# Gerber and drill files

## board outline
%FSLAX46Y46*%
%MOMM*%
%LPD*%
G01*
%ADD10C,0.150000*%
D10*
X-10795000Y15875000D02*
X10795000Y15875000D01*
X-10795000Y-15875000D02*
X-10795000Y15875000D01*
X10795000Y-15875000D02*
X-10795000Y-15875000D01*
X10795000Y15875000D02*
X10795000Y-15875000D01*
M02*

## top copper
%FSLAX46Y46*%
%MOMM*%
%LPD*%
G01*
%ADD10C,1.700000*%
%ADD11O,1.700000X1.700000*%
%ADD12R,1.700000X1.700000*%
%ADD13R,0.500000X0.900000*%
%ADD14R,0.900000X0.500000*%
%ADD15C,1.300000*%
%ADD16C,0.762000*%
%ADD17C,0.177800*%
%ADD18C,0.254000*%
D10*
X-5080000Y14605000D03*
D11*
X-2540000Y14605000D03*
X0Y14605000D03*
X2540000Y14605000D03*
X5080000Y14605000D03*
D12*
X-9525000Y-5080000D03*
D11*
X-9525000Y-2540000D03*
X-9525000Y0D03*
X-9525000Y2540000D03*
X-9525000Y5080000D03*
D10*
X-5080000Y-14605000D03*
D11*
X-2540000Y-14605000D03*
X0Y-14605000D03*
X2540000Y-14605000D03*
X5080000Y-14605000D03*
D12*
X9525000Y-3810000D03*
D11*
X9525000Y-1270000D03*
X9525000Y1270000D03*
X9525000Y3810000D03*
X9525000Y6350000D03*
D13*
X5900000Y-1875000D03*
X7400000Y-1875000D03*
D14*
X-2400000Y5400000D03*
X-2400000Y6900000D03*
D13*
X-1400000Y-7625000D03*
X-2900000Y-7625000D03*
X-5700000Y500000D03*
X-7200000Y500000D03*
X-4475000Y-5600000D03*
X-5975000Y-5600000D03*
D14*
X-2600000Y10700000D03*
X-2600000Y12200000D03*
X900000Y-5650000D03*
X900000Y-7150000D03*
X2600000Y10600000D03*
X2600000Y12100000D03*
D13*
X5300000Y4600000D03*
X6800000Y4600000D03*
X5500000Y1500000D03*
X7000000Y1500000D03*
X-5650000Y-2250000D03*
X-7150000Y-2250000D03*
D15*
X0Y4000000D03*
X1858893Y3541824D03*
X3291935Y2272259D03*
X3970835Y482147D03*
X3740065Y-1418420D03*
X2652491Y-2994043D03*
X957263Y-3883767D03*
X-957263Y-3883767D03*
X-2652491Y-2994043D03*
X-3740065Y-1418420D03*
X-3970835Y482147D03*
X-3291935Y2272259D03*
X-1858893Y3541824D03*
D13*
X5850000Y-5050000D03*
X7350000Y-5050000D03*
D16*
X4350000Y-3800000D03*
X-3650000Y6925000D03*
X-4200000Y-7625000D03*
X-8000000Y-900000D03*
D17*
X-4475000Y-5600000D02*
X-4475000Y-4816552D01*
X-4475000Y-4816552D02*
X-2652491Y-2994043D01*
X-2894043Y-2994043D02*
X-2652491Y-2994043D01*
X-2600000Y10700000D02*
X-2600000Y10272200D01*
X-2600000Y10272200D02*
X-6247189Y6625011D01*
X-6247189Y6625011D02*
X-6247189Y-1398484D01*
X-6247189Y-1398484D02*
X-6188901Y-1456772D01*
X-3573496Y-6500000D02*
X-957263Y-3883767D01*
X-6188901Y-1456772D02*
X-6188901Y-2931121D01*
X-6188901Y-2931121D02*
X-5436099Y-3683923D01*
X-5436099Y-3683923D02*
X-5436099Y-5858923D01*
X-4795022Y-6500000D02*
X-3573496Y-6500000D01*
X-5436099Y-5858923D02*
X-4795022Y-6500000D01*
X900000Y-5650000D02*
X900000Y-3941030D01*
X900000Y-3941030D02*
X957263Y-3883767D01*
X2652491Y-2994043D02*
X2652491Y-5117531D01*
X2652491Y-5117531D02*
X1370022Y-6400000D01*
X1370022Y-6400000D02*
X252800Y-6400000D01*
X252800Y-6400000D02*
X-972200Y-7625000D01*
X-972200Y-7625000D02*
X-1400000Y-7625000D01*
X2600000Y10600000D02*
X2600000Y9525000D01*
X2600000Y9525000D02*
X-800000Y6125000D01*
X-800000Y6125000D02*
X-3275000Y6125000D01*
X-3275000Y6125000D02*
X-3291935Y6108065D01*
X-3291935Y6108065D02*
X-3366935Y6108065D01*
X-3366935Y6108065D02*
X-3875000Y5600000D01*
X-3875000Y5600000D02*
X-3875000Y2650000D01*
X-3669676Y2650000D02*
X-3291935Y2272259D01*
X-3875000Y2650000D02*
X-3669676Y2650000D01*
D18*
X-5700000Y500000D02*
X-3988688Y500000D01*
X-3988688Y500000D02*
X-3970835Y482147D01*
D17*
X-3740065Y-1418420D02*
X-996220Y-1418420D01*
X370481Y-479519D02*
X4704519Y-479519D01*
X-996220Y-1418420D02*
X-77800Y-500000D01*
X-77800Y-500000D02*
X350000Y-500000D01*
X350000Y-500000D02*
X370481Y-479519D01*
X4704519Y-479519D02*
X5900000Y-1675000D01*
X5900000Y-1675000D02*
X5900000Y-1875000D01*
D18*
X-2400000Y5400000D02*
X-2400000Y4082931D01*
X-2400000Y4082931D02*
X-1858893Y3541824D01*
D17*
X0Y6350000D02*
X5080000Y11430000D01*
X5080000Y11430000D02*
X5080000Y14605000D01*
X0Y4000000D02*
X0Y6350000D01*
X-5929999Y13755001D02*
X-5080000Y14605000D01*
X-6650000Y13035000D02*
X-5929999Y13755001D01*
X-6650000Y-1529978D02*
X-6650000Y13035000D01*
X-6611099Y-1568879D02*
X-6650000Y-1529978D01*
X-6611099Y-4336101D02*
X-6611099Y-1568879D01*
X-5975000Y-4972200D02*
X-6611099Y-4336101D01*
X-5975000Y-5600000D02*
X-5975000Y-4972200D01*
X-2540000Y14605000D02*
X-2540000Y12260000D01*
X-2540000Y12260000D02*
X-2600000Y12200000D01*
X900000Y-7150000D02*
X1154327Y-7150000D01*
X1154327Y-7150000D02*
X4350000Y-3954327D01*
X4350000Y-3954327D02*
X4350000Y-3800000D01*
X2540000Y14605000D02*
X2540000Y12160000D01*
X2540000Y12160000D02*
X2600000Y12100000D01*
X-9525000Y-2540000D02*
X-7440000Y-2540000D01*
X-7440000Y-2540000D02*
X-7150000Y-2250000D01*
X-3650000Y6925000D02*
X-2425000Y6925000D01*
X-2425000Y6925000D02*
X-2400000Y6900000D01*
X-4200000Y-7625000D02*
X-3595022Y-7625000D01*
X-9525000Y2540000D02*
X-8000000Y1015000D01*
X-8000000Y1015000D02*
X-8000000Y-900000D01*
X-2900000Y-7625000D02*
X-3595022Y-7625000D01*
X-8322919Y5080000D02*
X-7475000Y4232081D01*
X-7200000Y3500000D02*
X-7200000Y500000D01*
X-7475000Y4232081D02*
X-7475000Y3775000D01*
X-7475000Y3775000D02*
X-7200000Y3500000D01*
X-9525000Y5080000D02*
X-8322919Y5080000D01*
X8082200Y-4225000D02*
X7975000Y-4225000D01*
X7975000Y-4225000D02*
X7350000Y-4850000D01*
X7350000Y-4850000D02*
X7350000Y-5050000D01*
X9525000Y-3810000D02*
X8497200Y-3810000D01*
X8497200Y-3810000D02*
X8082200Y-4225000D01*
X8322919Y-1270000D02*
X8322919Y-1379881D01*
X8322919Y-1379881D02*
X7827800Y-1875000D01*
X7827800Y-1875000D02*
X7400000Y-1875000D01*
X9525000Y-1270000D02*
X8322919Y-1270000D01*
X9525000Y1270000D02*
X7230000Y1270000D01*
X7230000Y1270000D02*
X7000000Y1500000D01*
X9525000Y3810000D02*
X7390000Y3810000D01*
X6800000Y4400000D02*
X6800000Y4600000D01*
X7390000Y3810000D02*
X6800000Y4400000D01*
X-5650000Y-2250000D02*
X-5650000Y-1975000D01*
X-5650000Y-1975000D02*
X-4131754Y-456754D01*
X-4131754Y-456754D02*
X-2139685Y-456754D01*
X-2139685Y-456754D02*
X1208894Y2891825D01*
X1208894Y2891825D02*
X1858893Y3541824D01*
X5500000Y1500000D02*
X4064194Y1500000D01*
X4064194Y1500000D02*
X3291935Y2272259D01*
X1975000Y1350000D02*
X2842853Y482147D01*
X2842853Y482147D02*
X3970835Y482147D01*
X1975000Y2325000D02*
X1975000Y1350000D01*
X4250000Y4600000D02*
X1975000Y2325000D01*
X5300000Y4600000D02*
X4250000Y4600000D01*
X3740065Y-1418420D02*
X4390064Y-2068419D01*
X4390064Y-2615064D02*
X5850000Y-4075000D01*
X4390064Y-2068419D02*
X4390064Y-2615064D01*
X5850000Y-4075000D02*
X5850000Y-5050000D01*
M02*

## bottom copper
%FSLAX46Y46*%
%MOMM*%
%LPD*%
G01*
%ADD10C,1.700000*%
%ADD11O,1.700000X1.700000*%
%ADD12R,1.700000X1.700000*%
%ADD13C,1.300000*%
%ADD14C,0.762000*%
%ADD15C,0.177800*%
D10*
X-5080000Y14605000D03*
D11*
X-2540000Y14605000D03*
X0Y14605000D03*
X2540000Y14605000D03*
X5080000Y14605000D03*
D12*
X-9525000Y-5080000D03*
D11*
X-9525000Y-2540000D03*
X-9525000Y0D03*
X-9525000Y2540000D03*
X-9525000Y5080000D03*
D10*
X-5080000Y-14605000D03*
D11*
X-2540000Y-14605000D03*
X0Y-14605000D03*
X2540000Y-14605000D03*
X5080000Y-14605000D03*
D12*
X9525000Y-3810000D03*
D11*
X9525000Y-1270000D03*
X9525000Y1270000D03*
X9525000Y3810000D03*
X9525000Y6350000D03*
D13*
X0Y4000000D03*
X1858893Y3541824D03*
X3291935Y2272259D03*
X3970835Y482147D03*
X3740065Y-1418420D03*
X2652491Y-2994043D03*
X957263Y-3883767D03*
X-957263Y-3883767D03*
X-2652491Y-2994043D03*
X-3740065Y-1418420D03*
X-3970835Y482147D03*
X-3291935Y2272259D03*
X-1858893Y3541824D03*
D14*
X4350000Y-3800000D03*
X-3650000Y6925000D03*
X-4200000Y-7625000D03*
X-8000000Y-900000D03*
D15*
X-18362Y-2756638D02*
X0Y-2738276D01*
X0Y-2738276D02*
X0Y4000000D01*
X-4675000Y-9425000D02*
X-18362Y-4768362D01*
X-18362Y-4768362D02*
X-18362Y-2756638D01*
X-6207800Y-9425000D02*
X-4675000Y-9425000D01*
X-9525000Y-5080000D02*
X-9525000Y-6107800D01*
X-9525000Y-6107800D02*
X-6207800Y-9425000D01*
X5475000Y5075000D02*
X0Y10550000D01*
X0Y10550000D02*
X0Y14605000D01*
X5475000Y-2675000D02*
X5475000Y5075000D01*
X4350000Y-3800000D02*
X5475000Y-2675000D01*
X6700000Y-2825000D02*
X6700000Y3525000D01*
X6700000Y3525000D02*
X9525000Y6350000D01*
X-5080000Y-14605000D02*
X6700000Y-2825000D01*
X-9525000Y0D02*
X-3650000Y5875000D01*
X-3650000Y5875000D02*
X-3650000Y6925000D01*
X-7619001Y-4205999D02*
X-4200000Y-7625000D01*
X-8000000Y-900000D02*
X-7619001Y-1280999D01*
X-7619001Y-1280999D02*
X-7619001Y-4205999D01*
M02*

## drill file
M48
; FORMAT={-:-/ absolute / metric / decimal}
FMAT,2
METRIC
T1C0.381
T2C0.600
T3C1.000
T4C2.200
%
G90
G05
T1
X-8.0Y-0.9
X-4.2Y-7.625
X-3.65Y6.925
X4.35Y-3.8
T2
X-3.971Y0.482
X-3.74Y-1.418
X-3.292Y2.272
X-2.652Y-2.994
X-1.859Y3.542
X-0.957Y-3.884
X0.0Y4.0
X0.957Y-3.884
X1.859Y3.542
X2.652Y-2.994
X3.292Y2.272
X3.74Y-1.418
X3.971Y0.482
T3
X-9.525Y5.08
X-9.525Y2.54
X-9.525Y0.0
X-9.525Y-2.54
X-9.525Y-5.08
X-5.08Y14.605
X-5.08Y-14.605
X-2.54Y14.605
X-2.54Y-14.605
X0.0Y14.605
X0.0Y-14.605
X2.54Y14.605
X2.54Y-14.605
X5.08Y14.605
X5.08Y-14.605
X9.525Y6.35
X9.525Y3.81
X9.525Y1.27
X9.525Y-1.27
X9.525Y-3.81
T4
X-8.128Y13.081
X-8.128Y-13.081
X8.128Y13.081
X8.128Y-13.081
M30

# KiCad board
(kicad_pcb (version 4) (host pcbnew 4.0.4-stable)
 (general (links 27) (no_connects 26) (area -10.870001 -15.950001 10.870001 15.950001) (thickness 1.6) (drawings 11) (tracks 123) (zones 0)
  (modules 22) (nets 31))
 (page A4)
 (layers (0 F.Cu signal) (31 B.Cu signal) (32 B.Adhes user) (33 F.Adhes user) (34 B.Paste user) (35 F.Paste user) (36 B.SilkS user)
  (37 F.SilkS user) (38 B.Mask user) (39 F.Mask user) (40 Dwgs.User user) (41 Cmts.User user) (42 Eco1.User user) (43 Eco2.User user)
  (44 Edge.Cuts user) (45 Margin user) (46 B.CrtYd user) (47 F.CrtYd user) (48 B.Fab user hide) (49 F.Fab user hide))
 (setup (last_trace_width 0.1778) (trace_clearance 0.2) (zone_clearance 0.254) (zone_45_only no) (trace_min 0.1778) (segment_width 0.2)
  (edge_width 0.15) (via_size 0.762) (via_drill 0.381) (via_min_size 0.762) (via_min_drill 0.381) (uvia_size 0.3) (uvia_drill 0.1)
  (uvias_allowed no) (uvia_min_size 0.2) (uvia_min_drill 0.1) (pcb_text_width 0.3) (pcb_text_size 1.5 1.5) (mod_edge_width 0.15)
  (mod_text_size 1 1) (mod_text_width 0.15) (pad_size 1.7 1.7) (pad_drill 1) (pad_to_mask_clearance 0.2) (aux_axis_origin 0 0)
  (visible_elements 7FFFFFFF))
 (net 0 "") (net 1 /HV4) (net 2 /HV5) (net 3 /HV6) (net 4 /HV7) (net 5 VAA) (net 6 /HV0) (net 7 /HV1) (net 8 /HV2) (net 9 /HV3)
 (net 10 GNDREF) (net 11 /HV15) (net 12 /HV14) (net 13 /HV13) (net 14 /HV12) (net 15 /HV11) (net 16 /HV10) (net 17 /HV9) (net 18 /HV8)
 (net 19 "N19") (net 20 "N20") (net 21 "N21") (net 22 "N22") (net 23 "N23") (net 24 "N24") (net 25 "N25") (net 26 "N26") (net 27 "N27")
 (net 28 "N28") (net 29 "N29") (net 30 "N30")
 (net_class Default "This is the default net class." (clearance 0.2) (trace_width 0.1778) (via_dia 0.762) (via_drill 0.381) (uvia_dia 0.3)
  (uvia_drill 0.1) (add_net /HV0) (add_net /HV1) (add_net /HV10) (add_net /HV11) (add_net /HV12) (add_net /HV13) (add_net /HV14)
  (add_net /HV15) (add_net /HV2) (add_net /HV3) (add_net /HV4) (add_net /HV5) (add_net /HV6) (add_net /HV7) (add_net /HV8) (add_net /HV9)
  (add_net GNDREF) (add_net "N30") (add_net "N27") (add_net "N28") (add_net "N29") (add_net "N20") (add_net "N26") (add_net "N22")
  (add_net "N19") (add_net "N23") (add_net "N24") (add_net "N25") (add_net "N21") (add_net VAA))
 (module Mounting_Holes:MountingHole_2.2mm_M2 (layer F.Cu) (at 8.128 13.081)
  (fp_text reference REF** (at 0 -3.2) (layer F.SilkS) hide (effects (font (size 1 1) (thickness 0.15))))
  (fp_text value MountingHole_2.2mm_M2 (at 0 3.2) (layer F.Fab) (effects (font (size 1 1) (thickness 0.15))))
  (pad 1 np_thru_hole circle (at 0 0) (size 2.2 2.2) (drill 2.2) (layers *.Cu *.Mask)))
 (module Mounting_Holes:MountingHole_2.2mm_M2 (layer F.Cu) (at 8.128 -13.081)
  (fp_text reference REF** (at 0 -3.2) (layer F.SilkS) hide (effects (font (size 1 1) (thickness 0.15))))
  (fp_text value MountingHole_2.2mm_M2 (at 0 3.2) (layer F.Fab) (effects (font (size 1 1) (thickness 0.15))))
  (pad 1 np_thru_hole circle (at 0 0) (size 2.2 2.2) (drill 2.2) (layers *.Cu *.Mask)))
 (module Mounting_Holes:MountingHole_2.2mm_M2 (layer F.Cu) (at -8.128 -13.081)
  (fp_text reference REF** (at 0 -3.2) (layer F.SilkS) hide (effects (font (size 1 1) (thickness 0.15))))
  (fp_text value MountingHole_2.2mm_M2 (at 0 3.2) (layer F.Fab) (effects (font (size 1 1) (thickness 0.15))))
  (pad 1 np_thru_hole circle (at 0 0) (size 2.2 2.2) (drill 2.2) (layers *.Cu *.Mask)))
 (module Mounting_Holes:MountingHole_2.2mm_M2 (layer F.Cu) (at -8.128 13.081)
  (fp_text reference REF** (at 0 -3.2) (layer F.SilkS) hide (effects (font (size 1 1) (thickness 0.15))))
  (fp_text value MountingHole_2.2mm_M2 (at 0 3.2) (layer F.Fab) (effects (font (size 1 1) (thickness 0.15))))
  (pad 1 np_thru_hole circle (at 0 0) (size 2.2 2.2) (drill 2.2) (layers *.Cu *.Mask)))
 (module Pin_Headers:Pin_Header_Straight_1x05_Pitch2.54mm (layer F.Cu) (at -5.08 -14.605 90)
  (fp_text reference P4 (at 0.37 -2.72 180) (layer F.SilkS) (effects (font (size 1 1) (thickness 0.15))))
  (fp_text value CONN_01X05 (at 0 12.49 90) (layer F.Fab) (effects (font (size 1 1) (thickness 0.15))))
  (pad 1 thru_hole circle (at 0 0 90) (size 1.7 1.7) (drill 1) (layers *.Cu *.Mask) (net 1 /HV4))
  (pad 2 thru_hole oval (at 0 2.54 90) (size 1.7 1.7) (drill 1) (layers *.Cu *.Mask) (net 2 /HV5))
  (pad 3 thru_hole oval (at 0 5.08 90) (size 1.7 1.7) (drill 1) (layers *.Cu *.Mask) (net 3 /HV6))
  (pad 4 thru_hole oval (at 0 7.62 90) (size 1.7 1.7) (drill 1) (layers *.Cu *.Mask) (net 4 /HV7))
  (pad 5 thru_hole oval (at 0 10.16 90) (size 1.7 1.7) (drill 1) (layers *.Cu *.Mask) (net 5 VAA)))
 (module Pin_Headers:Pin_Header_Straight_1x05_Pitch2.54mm (layer F.Cu) (at -9.525 5.08 180)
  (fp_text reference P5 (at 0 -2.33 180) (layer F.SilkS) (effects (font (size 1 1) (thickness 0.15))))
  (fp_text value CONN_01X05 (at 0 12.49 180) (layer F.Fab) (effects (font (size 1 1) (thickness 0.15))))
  (pad 1 thru_hole rect (at 0 0 180) (size 1.7 1.7) (drill 1) (layers *.Cu *.Mask) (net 5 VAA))
  (pad 2 thru_hole oval (at 0 2.54 180) (size 1.7 1.7) (drill 1) (layers *.Cu *.Mask) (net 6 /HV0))
  (pad 3 thru_hole oval (at 0 5.08 180) (size 1.7 1.7) (drill 1) (layers *.Cu *.Mask) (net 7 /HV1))
  (pad 4 thru_hole oval (at 0 7.62 180) (size 1.7 1.7) (drill 1) (layers *.Cu *.Mask) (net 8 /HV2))
  (pad 5 thru_hole oval (at 0 10.16 180) (size 1.7 1.7) (drill 1) (layers *.Cu *.Mask) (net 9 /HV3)))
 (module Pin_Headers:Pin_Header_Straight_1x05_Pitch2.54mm (layer F.Cu) (at -5.08 14.605 90)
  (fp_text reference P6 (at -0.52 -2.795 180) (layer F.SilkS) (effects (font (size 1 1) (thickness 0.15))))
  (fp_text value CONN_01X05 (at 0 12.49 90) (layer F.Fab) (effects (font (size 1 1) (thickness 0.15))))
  (pad 1 thru_hole circle (at 0 0 90) (size 1.7 1.7) (drill 1) (layers *.Cu *.Mask) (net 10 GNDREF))
  (pad 2 thru_hole oval (at 0 2.54 90) (size 1.7 1.7) (drill 1) (layers *.Cu *.Mask) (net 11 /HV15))
  (pad 3 thru_hole oval (at 0 5.08 90) (size 1.7 1.7) (drill 1) (layers *.Cu *.Mask) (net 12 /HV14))
  (pad 4 thru_hole oval (at 0 7.62 90) (size 1.7 1.7) (drill 1) (layers *.Cu *.Mask) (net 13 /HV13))
  (pad 5 thru_hole oval (at 0 10.16 90) (size 1.7 1.7) (drill 1) (layers *.Cu *.Mask) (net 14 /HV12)))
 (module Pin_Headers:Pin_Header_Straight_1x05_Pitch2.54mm (layer F.Cu) (at 9.525 3.81 180)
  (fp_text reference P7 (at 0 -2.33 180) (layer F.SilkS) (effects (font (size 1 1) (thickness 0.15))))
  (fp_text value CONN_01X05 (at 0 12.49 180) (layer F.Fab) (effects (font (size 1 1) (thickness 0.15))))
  (pad 1 thru_hole rect (at 0 0 180) (size 1.7 1.7) (drill 1) (layers *.Cu *.Mask) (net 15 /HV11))
  (pad 2 thru_hole oval (at 0 2.54 180) (size 1.7 1.7) (drill 1) (layers *.Cu *.Mask) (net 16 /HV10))
  (pad 3 thru_hole oval (at 0 5.08 180) (size 1.7 1.7) (drill 1) (layers *.Cu *.Mask) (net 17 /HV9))
  (pad 4 thru_hole oval (at 0 7.62 180) (size 1.7 1.7) (drill 1) (layers *.Cu *.Mask) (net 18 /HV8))
  (pad 5 thru_hole oval (at 0 10.16 180) (size 1.7 1.7) (drill 1) (layers *.Cu *.Mask) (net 10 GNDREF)))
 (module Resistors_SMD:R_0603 (layer F.Cu) (at 6.65 1.875)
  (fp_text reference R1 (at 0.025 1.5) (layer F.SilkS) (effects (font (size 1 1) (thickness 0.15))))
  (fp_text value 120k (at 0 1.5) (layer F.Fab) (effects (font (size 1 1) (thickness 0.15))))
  (pad 1 smd rect (at -0.75 0) (size 0.5 0.9) (layers F.Cu F.Paste F.Mask) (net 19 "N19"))
  (pad 2 smd rect (at 0.75 0) (size 0.5 0.9) (layers F.Cu F.Paste F.Mask) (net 16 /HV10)))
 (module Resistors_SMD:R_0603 (layer F.Cu) (at -2.4 -6.15 90)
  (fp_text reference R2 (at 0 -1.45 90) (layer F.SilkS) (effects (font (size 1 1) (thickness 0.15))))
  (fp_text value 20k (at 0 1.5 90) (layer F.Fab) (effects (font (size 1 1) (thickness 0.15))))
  (pad 1 smd rect (at -0.75 0 90) (size 0.5 0.9) (layers F.Cu F.Paste F.Mask) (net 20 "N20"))
  (pad 2 smd rect (at 0.75 0 90) (size 0.5 0.9) (layers F.Cu F.Paste F.Mask) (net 7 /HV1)))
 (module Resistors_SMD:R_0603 (layer F.Cu) (at -2.15 7.625 180)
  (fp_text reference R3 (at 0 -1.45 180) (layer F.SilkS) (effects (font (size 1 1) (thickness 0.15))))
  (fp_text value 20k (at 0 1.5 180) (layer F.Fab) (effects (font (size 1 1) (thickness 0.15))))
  (pad 1 smd rect (at -0.75 0 180) (size 0.5 0.9) (layers F.Cu F.Paste F.Mask) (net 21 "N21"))
  (pad 2 smd rect (at 0.75 0 180) (size 0.5 0.9) (layers F.Cu F.Paste F.Mask) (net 8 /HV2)))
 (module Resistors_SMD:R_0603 (layer F.Cu) (at -6.45 -0.5 180)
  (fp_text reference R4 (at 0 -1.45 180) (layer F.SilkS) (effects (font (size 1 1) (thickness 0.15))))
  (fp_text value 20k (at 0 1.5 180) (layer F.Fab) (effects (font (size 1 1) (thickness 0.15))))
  (pad 1 smd rect (at -0.75 0 180) (size 0.5 0.9) (layers F.Cu F.Paste F.Mask) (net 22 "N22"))
  (pad 2 smd rect (at 0.75 0 180) (size 0.5 0.9) (layers F.Cu F.Paste F.Mask) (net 9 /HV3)))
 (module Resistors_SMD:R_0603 (layer F.Cu) (at -5.225 5.6 180)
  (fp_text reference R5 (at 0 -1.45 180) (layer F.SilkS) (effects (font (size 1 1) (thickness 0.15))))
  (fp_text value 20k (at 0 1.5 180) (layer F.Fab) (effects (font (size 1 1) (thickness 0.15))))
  (pad 1 smd rect (at -0.75 0 180) (size 0.5 0.9) (layers F.Cu F.Paste F.Mask) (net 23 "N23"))
  (pad 2 smd rect (at 0.75 0 180) (size 0.5 0.9) (layers F.Cu F.Paste F.Mask) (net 1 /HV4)))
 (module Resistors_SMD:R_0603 (layer F.Cu) (at -2.6 -11.45 90)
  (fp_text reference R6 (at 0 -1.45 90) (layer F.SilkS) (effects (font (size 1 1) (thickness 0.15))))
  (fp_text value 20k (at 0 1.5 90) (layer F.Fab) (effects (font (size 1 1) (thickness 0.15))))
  (pad 1 smd rect (at -0.75 0 90) (size 0.5 0.9) (layers F.Cu F.Paste F.Mask) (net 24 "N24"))
  (pad 2 smd rect (at 0.75 0 90) (size 0.5 0.9) (layers F.Cu F.Paste F.Mask) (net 2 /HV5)))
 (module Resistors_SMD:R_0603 (layer F.Cu) (at 0.9 6.4 270)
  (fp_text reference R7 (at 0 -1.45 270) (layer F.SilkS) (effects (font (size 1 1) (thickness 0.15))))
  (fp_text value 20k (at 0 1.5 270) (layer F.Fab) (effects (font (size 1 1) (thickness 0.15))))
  (pad 1 smd rect (at -0.75 0 270) (size 0.5 0.9) (layers F.Cu F.Paste F.Mask) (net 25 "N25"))
  (pad 2 smd rect (at 0.75 0 270) (size 0.5 0.9) (layers F.Cu F.Paste F.Mask) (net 3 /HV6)))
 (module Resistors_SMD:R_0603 (layer F.Cu) (at 2.6 -11.35 90)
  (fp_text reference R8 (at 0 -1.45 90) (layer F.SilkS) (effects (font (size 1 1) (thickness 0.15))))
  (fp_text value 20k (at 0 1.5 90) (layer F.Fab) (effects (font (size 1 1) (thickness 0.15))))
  (pad 1 smd rect (at -0.75 0 90) (size 0.5 0.9) (layers F.Cu F.Paste F.Mask) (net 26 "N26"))
  (pad 2 smd rect (at 0.75 0 90) (size 0.5 0.9) (layers F.Cu F.Paste F.Mask) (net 4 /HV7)))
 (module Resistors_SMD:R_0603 (layer F.Cu) (at 6.05 -4.6)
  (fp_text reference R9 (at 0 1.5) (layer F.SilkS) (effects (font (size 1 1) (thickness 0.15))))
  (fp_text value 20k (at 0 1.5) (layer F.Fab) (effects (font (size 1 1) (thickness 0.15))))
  (pad 1 smd rect (at -0.75 0) (size 0.5 0.9) (layers F.Cu F.Paste F.Mask) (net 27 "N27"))
  (pad 2 smd rect (at 0.75 0) (size 0.5 0.9) (layers F.Cu F.Paste F.Mask) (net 18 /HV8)))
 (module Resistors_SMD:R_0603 (layer F.Cu) (at 6.25 -1.5)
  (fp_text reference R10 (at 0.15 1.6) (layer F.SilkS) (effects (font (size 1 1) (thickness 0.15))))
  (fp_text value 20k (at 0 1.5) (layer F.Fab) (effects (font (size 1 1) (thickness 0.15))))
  (pad 1 smd rect (at -0.75 0) (size 0.5 0.9) (layers F.Cu F.Paste F.Mask) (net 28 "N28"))
  (pad 2 smd rect (at 0.75 0) (size 0.5 0.9) (layers F.Cu F.Paste F.Mask) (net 17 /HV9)))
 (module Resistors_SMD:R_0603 (layer F.Cu) (at -6.4 2.25 180)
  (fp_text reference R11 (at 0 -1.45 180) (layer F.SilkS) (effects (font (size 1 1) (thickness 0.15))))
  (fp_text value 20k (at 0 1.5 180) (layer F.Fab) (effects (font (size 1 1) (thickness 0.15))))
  (pad 1 smd rect (at -0.75 0 180) (size 0.5 0.9) (layers F.Cu F.Paste F.Mask) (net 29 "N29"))
  (pad 2 smd rect (at 0.75 0 180) (size 0.5 0.9) (layers F.Cu F.Paste F.Mask) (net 6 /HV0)))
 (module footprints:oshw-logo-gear (layer B.Cu) (at 6.9342 -9.652 180)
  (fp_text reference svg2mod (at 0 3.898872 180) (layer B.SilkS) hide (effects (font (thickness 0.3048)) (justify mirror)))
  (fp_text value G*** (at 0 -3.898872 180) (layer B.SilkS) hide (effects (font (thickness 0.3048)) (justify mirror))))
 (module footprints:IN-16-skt (layer B.Cu) (at 0 0 180)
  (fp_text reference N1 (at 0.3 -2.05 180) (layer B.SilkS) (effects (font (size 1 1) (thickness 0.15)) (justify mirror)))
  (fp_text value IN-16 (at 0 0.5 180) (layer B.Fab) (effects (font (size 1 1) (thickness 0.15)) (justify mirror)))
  (pad 1 thru_hole circle (at 0 4 180) (size 1.3 1.3) (drill 0.6) (layers *.Cu *.Mask) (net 5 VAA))
  (pad 13 thru_hole circle (at -1.858893 3.541824 152.3077) (size 1.3 1.3) (drill 0.6) (layers *.Cu *.Mask) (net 29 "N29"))
  (pad 12 thru_hole circle (at -3.291935 2.272259 124.6154) (size 1.3 1.3) (drill 0.6) (layers *.Cu *.Mask) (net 28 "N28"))
  (pad 11 thru_hole circle (at -3.970835 0.482147 96.9231) (size 1.3 1.3) (drill 0.6) (layers *.Cu *.Mask) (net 27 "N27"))
  (pad 10 thru_hole circle (at -3.740065 -1.41842 69.231) (size 1.3 1.3) (drill 0.6) (layers *.Cu *.Mask) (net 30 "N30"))
  (pad 9 thru_hole circle (at -2.652491 -2.994043 41.538) (size 1.3 1.3) (drill 0.6) (layers *.Cu *.Mask) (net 21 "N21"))
  (pad 8 thru_hole circle (at -0.957263 -3.883767 13.846) (size 1.3 1.3) (drill 0.6) (layers *.Cu *.Mask) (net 25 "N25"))
  (pad 7 thru_hole circle (at 0.957263 -3.883767 346.154) (size 1.3 1.3) (drill 0.6) (layers *.Cu *.Mask) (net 24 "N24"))
  (pad 6 thru_hole circle (at 2.652491 -2.994043 318.462) (size 1.3 1.3) (drill 0.6) (layers *.Cu *.Mask) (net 23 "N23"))
  (pad 5 thru_hole circle (at 3.740065 -1.41842 290.769) (size 1.3 1.3) (drill 0.6) (layers *.Cu *.Mask) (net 19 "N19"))
  (pad 4 thru_hole circle (at 3.970835 0.482147 263.0769) (size 1.3 1.3) (drill 0.6) (layers *.Cu *.Mask) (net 22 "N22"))
  (pad 3 thru_hole circle (at 3.291935 2.272259 235.3846) (size 1.3 1.3) (drill 0.6) (layers *.Cu *.Mask) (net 26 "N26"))
  (pad 2 thru_hole circle (at 1.858893 3.541824 207.6923) (size 1.3 1.3) (drill 0.6) (layers *.Cu *.Mask) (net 20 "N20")))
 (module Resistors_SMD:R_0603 (layer F.Cu) (at 6.6 5.05)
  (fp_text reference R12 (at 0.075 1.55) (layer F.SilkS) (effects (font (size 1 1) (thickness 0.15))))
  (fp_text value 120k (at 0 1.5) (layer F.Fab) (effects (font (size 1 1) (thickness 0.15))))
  (pad 1 smd rect (at -0.75 0) (size 0.5 0.9) (layers F.Cu F.Paste F.Mask) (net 30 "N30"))
  (pad 2 smd rect (at 0.75 0) (size 0.5 0.9) (layers F.Cu F.Paste F.Mask) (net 15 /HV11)))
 (gr_line (start -10.795 -15.875) (end 10.795 -15.875) (layer Edge.Cuts) (width 0.15))
 (gr_line (start -10.795 15.875) (end -10.795 -15.875) (layer Edge.Cuts) (width 0.15))
 (gr_line (start 10.795 15.875) (end -10.795 15.875) (layer Edge.Cuts) (width 0.15))
 (gr_line (start 10.795 -15.875) (end 10.795 15.875) (layer Edge.Cuts) (width 0.15))
 (segment (start -4.475 5.6) (end -4.475 4.816552) (width 0.1778) (layer F.Cu) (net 23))
 (segment (start -4.475 4.816552) (end -2.652491 2.994043) (width 0.1778) (layer F.Cu) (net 23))
 (segment (start -2.894043 2.994043) (end -2.652491 2.994043) (width 0.1778) (layer F.Cu) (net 23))
 (segment (start -2.6 -10.7) (end -2.6 -10.2722) (width 0.1778) (layer F.Cu) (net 24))
 (segment (start -2.6 -10.2722) (end -6.247189 -6.625011) (width 0.1778) (layer F.Cu) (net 24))
 (segment (start -6.247189 -6.625011) (end -6.247189 1.398484) (width 0.1778) (layer F.Cu) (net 24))
 (segment (start -6.247189 1.398484) (end -6.188901 1.456772) (width 0.1778) (layer F.Cu) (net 24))
 (segment (start -3.573496 6.5) (end -0.957263 3.883767) (width 0.1778) (layer F.Cu) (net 24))
 (segment (start -6.188901 1.456772) (end -6.188901 2.931121) (width 0.1778) (layer F.Cu) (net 24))
 (segment (start -6.188901 2.931121) (end -5.436099 3.683923) (width 0.1778) (layer F.Cu) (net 24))
 (segment (start -5.436099 3.683923) (end -5.436099 5.858923) (width 0.1778) (layer F.Cu) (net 24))
 (segment (start -4.795022 6.5) (end -3.573496 6.5) (width 0.1778) (layer F.Cu) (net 24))
 (segment (start -5.436099 5.858923) (end -4.795022 6.5) (width 0.1778) (layer F.Cu) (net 24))
 (segment (start 0.9 5.65) (end 0.9 3.94103) (width 0.1778) (layer F.Cu) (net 25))
 (segment (start 0.9 3.94103) (end 0.957263 3.883767) (width 0.1778) (layer F.Cu) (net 25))
 (segment (start 2.652491 2.994043) (end 2.652491 5.117531) (width 0.1778) (layer F.Cu) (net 21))
 (segment (start 2.652491 5.117531) (end 1.370022 6.4) (width 0.1778) (layer F.Cu) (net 21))
 (segment (start 1.370022 6.4) (end 0.2528 6.4) (width 0.1778) (layer F.Cu) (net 21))
 (segment (start 0.2528 6.4) (end -0.9722 7.625) (width 0.1778) (layer F.Cu) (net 21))
 (segment (start -0.9722 7.625) (end -1.4 7.625) (width 0.1778) (layer F.Cu) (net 21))
 (segment (start 2.6 -10.6) (end 2.6 -9.525) (width 0.1778) (layer F.Cu) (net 26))
 (segment (start 2.6 -9.525) (end -0.8 -6.125) (width 0.1778) (layer F.Cu) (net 26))
 (segment (start -0.8 -6.125) (end -3.275 -6.125) (width 0.1778) (layer F.Cu) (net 26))
 (segment (start -3.275 -6.125) (end -3.291935 -6.108065) (width 0.1778) (layer F.Cu) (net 26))
 (segment (start -3.291935 -6.108065) (end -3.366935 -6.108065) (width 0.1778) (layer F.Cu) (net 26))
 (segment (start -3.366935 -6.108065) (end -3.875 -5.6) (width 0.1778) (layer F.Cu) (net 26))
 (segment (start -3.875 -5.6) (end -3.875 -2.65) (width 0.1778) (layer F.Cu) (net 26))
 (segment (start -3.669676 -2.65) (end -3.291935 -2.272259) (width 0.1778) (layer F.Cu) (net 26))
 (segment (start -3.875 -2.65) (end -3.669676 -2.65) (width 0.1778) (layer F.Cu) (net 26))
 (segment (start -5.7 -0.5) (end -3.988688 -0.5) (width 0.254) (layer F.Cu) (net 22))
 (segment (start -3.988688 -0.5) (end -3.970835 -0.482147) (width 0.254) (layer F.Cu) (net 22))
 (segment (start -3.740065 1.41842) (end -0.99622 1.41842) (width 0.1778) (layer F.Cu) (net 19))
 (segment (start 0.370481 0.479519) (end 4.704519 0.479519) (width 0.1778) (layer F.Cu) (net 19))
 (segment (start -0.99622 1.41842) (end -0.0778 0.5) (width 0.1778) (layer F.Cu) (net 19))
 (segment (start -0.0778 0.5) (end 0.35 0.5) (width 0.1778) (layer F.Cu) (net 19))
 (segment (start 0.35 0.5) (end 0.370481 0.479519) (width 0.1778) (layer F.Cu) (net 19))
 (segment (start 4.704519 0.479519) (end 5.9 1.675) (width 0.1778) (layer F.Cu) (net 19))
 (segment (start 5.9 1.675) (end 5.9 1.875) (width 0.1778) (layer F.Cu) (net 19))
 (segment (start -2.4 -5.4) (end -2.4 -4.082931) (width 0.254) (layer F.Cu) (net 20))
 (segment (start -2.4 -4.082931) (end -1.858893 -3.541824) (width 0.254) (layer F.Cu) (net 20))
 (segment (start -0.018362 2.756638) (end 0 2.738276) (width 0.1778) (layer B.Cu) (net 5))
 (segment (start 0 2.738276) (end 0 -4) (width 0.1778) (layer B.Cu) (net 5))
 (segment (start -4.675 9.425) (end -0.018362 4.768362) (width 0.1778) (layer B.Cu) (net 5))
 (segment (start -0.018362 4.768362) (end -0.018362 2.756638) (width 0.1778) (layer B.Cu) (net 5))
 (segment (start -6.2078 9.425) (end -4.675 9.425) (width 0.1778) (layer B.Cu) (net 5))
 (segment (start -9.525 5.08) (end -9.525 6.1078) (width 0.1778) (layer B.Cu) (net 5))
 (segment (start -9.525 6.1078) (end -6.2078 9.425) (width 0.1778) (layer B.Cu) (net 5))
 (segment (start 0 -6.35) (end 5.08 -11.43) (width 0.1778) (layer F.Cu) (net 5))
 (segment (start 5.08 -11.43) (end 5.08 -14.605) (width 0.1778) (layer F.Cu) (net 5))
 (segment (start 0 -4) (end 0 -6.35) (width 0.1778) (layer F.Cu) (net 5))
 (segment (start -5.929999 -13.755001) (end -5.08 -14.605) (width 0.1778) (layer F.Cu) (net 1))
 (segment (start -6.65 -13.035) (end -5.929999 -13.755001) (width 0.1778) (layer F.Cu) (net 1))
 (segment (start -6.65 1.529978) (end -6.65 -13.035) (width 0.1778) (layer F.Cu) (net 1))
 (segment (start -6.611099 1.568879) (end -6.65 1.529978) (width 0.1778) (layer F.Cu) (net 1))
 (segment (start -6.611099 4.336101) (end -6.611099 1.568879) (width 0.1778) (layer F.Cu) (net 1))
 (segment (start -5.975 4.9722) (end -6.611099 4.336101) (width 0.1778) (layer F.Cu) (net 1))
 (segment (start -5.975 5.6) (end -5.975 4.9722) (width 0.1778) (layer F.Cu) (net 1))
 (segment (start -2.54 -14.605) (end -2.54 -12.26) (width 0.1778) (layer F.Cu) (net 2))
 (segment (start -2.54 -12.26) (end -2.6 -12.2) (width 0.1778) (layer F.Cu) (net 2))
 (segment (start 5.475 -5.075) (end 0 -10.55) (width 0.1778) (layer B.Cu) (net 3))
 (segment (start 0 -10.55) (end 0 -14.605) (width 0.1778) (layer B.Cu) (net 3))
 (segment (start 5.475 2.675) (end 5.475 -5.075) (width 0.1778) (layer B.Cu) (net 3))
 (segment (start 4.35 3.8) (end 5.475 2.675) (width 0.1778) (layer B.Cu) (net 3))
 (segment (start 0.9 7.15) (end 1.154327 7.15) (width 0.1778) (layer F.Cu) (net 3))
 (segment (start 1.154327 7.15) (end 4.35 3.954327) (width 0.1778) (layer F.Cu) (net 3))
 (segment (start 4.35 3.954327) (end 4.35 3.8) (width 0.1778) (layer F.Cu) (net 3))
 (via (at 4.35 3.8) (size 0.762) (drill 0.381) (layers F.Cu B.Cu) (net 3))
 (segment (start 2.54 -14.605) (end 2.54 -12.16) (width 0.1778) (layer F.Cu) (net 4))
 (segment (start 2.54 -12.16) (end 2.6 -12.1) (width 0.1778) (layer F.Cu) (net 4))
 (segment (start 6.7 2.825) (end 6.7 -3.525) (width 0.1778) (layer B.Cu) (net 10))
 (segment (start 6.7 -3.525) (end 9.525 -6.35) (width 0.1778) (layer B.Cu) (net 10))
 (segment (start -5.08 14.605) (end 6.7 2.825) (width 0.1778) (layer B.Cu) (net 10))
 (segment (start -9.525 2.54) (end -7.44 2.54) (width 0.1778) (layer F.Cu) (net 6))
 (segment (start -7.44 2.54) (end -7.15 2.25) (width 0.1778) (layer F.Cu) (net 6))
 (segment (start -3.65 -6.925) (end -2.425 -6.925) (width 0.1778) (layer F.Cu) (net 7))
 (segment (start -2.425 -6.925) (end -2.4 -6.9) (width 0.1778) (layer F.Cu) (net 7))
 (segment (start -9.525 0) (end -3.65 -5.875) (width 0.1778) (layer B.Cu) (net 7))
 (segment (start -3.65 -5.875) (end -3.65 -6.925) (width 0.1778) (layer B.Cu) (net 7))
 (via (at -3.65 -6.925) (size 0.762) (drill 0.381) (layers F.Cu B.Cu) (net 7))
 (segment (start -4.2 7.625) (end -3.595022 7.625) (width 0.1778) (layer F.Cu) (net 8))
 (segment (start -7.619001 4.205999) (end -4.2 7.625) (width 0.1778) (layer B.Cu) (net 8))
 (via (at -4.2 7.625) (size 0.762) (drill 0.381) (layers F.Cu B.Cu) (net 8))
 (segment (start -8 0.9) (end -7.619001 1.280999) (width 0.1778) (layer B.Cu) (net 8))
 (segment (start -7.619001 1.280999) (end -7.619001 4.205999) (width 0.1778) (layer B.Cu) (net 8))
 (segment (start -9.525 -2.54) (end -8 -1.015) (width 0.1778) (layer F.Cu) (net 8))
 (segment (start -8 -1.015) (end -8 0.9) (width 0.1778) (layer F.Cu) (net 8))
 (via (at -8 0.9) (size 0.762) (drill 0.381) (layers F.Cu B.Cu) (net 8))
 (segment (start -2.9 7.625) (end -3.595022 7.625) (width 0.1778) (layer F.Cu) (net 8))
 (segment (start -8.322919 -5.08) (end -7.475 -4.232081) (width 0.1778) (layer F.Cu) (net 9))
 (segment (start -7.2 -3.5) (end -7.2 -0.5) (width 0.1778) (layer F.Cu) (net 9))
 (segment (start -7.475 -4.232081) (end -7.475 -3.775) (width 0.1778) (layer F.Cu) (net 9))
 (segment (start -7.475 -3.775) (end -7.2 -3.5) (width 0.1778) (layer F.Cu) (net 9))
 (segment (start -9.525 -5.08) (end -8.322919 -5.08) (width 0.1778) (layer F.Cu) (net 9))
 (segment (start 8.0822 4.225) (end 7.975 4.225) (width 0.1778) (layer F.Cu) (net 15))
 (segment (start 7.975 4.225) (end 7.35 4.85) (width 0.1778) (layer F.Cu) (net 15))
 (segment (start 7.35 4.85) (end 7.35 5.05) (width 0.1778) (layer F.Cu) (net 15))
 (segment (start 9.525 3.81) (end 8.4972 3.81) (width 0.1778) (layer F.Cu) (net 15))
 (segment (start 8.4972 3.81) (end 8.0822 4.225) (width 0.1778) (layer F.Cu) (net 15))
 (segment (start 8.322919 1.27) (end 8.322919 1.379881) (width 0.1778) (layer F.Cu) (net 16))
 (segment (start 8.322919 1.379881) (end 7.8278 1.875) (width 0.1778) (layer F.Cu) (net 16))
 (segment (start 7.8278 1.875) (end 7.4 1.875) (width 0.1778) (layer F.Cu) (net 16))
 (segment (start 9.525 1.27) (end 8.322919 1.27) (width 0.1778) (layer F.Cu) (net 16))
 (segment (start 9.525 -1.27) (end 7.23 -1.27) (width 0.1778) (layer F.Cu) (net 17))
 (segment (start 7.23 -1.27) (end 7 -1.5) (width 0.1778) (layer F.Cu) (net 17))
 (segment (start 9.525 -3.81) (end 7.39 -3.81) (width 0.1778) (layer F.Cu) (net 18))
 (segment (start 6.8 -4.4) (end 6.8 -4.6) (width 0.1778) (layer F.Cu) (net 18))
 (segment (start 7.39 -3.81) (end 6.8 -4.4) (width 0.1778) (layer F.Cu) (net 18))
 (segment (start -5.65 2.25) (end -5.65 1.975) (width 0.1778) (layer F.Cu) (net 29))
 (segment (start -5.65 1.975) (end -4.131754 0.456754) (width 0.1778) (layer F.Cu) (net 29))
 (segment (start -4.131754 0.456754) (end -2.139685 0.456754) (width 0.1778) (layer F.Cu) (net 29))
 (segment (start -2.139685 0.456754) (end 1.208894 -2.891825) (width 0.1778) (layer F.Cu) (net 29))
 (segment (start 1.208894 -2.891825) (end 1.858893 -3.541824) (width 0.1778) (layer F.Cu) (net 29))
 (segment (start 5.5 -1.5) (end 4.064194 -1.5) (width 0.1778) (layer F.Cu) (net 28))
 (segment (start 4.064194 -1.5) (end 3.291935 -2.272259) (width 0.1778) (layer F.Cu) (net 28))
 (segment (start 1.975 -1.35) (end 2.842853 -0.482147) (width 0.1778) (layer F.Cu) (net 27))
 (segment (start 2.842853 -0.482147) (end 3.970835 -0.482147) (width 0.1778) (layer F.Cu) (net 27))
 (segment (start 1.975 -2.325) (end 1.975 -1.35) (width 0.1778) (layer F.Cu) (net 27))
 (segment (start 4.25 -4.6) (end 1.975 -2.325) (width 0.1778) (layer F.Cu) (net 27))
 (segment (start 5.3 -4.6) (end 4.25 -4.6) (width 0.1778) (layer F.Cu) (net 27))
 (segment (start 3.740065 1.41842) (end 4.390064 2.068419) (width 0.1778) (layer F.Cu) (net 30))
 (segment (start 4.390064 2.615064) (end 5.85 4.075) (width 0.1778) (layer F.Cu) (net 30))
 (segment (start 4.390064 2.068419) (end 4.390064 2.615064) (width 0.1778) (layer F.Cu) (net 30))
 (segment (start 5.85 4.075) (end 5.85 5.05) (width 0.1778) (layer F.Cu) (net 30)))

